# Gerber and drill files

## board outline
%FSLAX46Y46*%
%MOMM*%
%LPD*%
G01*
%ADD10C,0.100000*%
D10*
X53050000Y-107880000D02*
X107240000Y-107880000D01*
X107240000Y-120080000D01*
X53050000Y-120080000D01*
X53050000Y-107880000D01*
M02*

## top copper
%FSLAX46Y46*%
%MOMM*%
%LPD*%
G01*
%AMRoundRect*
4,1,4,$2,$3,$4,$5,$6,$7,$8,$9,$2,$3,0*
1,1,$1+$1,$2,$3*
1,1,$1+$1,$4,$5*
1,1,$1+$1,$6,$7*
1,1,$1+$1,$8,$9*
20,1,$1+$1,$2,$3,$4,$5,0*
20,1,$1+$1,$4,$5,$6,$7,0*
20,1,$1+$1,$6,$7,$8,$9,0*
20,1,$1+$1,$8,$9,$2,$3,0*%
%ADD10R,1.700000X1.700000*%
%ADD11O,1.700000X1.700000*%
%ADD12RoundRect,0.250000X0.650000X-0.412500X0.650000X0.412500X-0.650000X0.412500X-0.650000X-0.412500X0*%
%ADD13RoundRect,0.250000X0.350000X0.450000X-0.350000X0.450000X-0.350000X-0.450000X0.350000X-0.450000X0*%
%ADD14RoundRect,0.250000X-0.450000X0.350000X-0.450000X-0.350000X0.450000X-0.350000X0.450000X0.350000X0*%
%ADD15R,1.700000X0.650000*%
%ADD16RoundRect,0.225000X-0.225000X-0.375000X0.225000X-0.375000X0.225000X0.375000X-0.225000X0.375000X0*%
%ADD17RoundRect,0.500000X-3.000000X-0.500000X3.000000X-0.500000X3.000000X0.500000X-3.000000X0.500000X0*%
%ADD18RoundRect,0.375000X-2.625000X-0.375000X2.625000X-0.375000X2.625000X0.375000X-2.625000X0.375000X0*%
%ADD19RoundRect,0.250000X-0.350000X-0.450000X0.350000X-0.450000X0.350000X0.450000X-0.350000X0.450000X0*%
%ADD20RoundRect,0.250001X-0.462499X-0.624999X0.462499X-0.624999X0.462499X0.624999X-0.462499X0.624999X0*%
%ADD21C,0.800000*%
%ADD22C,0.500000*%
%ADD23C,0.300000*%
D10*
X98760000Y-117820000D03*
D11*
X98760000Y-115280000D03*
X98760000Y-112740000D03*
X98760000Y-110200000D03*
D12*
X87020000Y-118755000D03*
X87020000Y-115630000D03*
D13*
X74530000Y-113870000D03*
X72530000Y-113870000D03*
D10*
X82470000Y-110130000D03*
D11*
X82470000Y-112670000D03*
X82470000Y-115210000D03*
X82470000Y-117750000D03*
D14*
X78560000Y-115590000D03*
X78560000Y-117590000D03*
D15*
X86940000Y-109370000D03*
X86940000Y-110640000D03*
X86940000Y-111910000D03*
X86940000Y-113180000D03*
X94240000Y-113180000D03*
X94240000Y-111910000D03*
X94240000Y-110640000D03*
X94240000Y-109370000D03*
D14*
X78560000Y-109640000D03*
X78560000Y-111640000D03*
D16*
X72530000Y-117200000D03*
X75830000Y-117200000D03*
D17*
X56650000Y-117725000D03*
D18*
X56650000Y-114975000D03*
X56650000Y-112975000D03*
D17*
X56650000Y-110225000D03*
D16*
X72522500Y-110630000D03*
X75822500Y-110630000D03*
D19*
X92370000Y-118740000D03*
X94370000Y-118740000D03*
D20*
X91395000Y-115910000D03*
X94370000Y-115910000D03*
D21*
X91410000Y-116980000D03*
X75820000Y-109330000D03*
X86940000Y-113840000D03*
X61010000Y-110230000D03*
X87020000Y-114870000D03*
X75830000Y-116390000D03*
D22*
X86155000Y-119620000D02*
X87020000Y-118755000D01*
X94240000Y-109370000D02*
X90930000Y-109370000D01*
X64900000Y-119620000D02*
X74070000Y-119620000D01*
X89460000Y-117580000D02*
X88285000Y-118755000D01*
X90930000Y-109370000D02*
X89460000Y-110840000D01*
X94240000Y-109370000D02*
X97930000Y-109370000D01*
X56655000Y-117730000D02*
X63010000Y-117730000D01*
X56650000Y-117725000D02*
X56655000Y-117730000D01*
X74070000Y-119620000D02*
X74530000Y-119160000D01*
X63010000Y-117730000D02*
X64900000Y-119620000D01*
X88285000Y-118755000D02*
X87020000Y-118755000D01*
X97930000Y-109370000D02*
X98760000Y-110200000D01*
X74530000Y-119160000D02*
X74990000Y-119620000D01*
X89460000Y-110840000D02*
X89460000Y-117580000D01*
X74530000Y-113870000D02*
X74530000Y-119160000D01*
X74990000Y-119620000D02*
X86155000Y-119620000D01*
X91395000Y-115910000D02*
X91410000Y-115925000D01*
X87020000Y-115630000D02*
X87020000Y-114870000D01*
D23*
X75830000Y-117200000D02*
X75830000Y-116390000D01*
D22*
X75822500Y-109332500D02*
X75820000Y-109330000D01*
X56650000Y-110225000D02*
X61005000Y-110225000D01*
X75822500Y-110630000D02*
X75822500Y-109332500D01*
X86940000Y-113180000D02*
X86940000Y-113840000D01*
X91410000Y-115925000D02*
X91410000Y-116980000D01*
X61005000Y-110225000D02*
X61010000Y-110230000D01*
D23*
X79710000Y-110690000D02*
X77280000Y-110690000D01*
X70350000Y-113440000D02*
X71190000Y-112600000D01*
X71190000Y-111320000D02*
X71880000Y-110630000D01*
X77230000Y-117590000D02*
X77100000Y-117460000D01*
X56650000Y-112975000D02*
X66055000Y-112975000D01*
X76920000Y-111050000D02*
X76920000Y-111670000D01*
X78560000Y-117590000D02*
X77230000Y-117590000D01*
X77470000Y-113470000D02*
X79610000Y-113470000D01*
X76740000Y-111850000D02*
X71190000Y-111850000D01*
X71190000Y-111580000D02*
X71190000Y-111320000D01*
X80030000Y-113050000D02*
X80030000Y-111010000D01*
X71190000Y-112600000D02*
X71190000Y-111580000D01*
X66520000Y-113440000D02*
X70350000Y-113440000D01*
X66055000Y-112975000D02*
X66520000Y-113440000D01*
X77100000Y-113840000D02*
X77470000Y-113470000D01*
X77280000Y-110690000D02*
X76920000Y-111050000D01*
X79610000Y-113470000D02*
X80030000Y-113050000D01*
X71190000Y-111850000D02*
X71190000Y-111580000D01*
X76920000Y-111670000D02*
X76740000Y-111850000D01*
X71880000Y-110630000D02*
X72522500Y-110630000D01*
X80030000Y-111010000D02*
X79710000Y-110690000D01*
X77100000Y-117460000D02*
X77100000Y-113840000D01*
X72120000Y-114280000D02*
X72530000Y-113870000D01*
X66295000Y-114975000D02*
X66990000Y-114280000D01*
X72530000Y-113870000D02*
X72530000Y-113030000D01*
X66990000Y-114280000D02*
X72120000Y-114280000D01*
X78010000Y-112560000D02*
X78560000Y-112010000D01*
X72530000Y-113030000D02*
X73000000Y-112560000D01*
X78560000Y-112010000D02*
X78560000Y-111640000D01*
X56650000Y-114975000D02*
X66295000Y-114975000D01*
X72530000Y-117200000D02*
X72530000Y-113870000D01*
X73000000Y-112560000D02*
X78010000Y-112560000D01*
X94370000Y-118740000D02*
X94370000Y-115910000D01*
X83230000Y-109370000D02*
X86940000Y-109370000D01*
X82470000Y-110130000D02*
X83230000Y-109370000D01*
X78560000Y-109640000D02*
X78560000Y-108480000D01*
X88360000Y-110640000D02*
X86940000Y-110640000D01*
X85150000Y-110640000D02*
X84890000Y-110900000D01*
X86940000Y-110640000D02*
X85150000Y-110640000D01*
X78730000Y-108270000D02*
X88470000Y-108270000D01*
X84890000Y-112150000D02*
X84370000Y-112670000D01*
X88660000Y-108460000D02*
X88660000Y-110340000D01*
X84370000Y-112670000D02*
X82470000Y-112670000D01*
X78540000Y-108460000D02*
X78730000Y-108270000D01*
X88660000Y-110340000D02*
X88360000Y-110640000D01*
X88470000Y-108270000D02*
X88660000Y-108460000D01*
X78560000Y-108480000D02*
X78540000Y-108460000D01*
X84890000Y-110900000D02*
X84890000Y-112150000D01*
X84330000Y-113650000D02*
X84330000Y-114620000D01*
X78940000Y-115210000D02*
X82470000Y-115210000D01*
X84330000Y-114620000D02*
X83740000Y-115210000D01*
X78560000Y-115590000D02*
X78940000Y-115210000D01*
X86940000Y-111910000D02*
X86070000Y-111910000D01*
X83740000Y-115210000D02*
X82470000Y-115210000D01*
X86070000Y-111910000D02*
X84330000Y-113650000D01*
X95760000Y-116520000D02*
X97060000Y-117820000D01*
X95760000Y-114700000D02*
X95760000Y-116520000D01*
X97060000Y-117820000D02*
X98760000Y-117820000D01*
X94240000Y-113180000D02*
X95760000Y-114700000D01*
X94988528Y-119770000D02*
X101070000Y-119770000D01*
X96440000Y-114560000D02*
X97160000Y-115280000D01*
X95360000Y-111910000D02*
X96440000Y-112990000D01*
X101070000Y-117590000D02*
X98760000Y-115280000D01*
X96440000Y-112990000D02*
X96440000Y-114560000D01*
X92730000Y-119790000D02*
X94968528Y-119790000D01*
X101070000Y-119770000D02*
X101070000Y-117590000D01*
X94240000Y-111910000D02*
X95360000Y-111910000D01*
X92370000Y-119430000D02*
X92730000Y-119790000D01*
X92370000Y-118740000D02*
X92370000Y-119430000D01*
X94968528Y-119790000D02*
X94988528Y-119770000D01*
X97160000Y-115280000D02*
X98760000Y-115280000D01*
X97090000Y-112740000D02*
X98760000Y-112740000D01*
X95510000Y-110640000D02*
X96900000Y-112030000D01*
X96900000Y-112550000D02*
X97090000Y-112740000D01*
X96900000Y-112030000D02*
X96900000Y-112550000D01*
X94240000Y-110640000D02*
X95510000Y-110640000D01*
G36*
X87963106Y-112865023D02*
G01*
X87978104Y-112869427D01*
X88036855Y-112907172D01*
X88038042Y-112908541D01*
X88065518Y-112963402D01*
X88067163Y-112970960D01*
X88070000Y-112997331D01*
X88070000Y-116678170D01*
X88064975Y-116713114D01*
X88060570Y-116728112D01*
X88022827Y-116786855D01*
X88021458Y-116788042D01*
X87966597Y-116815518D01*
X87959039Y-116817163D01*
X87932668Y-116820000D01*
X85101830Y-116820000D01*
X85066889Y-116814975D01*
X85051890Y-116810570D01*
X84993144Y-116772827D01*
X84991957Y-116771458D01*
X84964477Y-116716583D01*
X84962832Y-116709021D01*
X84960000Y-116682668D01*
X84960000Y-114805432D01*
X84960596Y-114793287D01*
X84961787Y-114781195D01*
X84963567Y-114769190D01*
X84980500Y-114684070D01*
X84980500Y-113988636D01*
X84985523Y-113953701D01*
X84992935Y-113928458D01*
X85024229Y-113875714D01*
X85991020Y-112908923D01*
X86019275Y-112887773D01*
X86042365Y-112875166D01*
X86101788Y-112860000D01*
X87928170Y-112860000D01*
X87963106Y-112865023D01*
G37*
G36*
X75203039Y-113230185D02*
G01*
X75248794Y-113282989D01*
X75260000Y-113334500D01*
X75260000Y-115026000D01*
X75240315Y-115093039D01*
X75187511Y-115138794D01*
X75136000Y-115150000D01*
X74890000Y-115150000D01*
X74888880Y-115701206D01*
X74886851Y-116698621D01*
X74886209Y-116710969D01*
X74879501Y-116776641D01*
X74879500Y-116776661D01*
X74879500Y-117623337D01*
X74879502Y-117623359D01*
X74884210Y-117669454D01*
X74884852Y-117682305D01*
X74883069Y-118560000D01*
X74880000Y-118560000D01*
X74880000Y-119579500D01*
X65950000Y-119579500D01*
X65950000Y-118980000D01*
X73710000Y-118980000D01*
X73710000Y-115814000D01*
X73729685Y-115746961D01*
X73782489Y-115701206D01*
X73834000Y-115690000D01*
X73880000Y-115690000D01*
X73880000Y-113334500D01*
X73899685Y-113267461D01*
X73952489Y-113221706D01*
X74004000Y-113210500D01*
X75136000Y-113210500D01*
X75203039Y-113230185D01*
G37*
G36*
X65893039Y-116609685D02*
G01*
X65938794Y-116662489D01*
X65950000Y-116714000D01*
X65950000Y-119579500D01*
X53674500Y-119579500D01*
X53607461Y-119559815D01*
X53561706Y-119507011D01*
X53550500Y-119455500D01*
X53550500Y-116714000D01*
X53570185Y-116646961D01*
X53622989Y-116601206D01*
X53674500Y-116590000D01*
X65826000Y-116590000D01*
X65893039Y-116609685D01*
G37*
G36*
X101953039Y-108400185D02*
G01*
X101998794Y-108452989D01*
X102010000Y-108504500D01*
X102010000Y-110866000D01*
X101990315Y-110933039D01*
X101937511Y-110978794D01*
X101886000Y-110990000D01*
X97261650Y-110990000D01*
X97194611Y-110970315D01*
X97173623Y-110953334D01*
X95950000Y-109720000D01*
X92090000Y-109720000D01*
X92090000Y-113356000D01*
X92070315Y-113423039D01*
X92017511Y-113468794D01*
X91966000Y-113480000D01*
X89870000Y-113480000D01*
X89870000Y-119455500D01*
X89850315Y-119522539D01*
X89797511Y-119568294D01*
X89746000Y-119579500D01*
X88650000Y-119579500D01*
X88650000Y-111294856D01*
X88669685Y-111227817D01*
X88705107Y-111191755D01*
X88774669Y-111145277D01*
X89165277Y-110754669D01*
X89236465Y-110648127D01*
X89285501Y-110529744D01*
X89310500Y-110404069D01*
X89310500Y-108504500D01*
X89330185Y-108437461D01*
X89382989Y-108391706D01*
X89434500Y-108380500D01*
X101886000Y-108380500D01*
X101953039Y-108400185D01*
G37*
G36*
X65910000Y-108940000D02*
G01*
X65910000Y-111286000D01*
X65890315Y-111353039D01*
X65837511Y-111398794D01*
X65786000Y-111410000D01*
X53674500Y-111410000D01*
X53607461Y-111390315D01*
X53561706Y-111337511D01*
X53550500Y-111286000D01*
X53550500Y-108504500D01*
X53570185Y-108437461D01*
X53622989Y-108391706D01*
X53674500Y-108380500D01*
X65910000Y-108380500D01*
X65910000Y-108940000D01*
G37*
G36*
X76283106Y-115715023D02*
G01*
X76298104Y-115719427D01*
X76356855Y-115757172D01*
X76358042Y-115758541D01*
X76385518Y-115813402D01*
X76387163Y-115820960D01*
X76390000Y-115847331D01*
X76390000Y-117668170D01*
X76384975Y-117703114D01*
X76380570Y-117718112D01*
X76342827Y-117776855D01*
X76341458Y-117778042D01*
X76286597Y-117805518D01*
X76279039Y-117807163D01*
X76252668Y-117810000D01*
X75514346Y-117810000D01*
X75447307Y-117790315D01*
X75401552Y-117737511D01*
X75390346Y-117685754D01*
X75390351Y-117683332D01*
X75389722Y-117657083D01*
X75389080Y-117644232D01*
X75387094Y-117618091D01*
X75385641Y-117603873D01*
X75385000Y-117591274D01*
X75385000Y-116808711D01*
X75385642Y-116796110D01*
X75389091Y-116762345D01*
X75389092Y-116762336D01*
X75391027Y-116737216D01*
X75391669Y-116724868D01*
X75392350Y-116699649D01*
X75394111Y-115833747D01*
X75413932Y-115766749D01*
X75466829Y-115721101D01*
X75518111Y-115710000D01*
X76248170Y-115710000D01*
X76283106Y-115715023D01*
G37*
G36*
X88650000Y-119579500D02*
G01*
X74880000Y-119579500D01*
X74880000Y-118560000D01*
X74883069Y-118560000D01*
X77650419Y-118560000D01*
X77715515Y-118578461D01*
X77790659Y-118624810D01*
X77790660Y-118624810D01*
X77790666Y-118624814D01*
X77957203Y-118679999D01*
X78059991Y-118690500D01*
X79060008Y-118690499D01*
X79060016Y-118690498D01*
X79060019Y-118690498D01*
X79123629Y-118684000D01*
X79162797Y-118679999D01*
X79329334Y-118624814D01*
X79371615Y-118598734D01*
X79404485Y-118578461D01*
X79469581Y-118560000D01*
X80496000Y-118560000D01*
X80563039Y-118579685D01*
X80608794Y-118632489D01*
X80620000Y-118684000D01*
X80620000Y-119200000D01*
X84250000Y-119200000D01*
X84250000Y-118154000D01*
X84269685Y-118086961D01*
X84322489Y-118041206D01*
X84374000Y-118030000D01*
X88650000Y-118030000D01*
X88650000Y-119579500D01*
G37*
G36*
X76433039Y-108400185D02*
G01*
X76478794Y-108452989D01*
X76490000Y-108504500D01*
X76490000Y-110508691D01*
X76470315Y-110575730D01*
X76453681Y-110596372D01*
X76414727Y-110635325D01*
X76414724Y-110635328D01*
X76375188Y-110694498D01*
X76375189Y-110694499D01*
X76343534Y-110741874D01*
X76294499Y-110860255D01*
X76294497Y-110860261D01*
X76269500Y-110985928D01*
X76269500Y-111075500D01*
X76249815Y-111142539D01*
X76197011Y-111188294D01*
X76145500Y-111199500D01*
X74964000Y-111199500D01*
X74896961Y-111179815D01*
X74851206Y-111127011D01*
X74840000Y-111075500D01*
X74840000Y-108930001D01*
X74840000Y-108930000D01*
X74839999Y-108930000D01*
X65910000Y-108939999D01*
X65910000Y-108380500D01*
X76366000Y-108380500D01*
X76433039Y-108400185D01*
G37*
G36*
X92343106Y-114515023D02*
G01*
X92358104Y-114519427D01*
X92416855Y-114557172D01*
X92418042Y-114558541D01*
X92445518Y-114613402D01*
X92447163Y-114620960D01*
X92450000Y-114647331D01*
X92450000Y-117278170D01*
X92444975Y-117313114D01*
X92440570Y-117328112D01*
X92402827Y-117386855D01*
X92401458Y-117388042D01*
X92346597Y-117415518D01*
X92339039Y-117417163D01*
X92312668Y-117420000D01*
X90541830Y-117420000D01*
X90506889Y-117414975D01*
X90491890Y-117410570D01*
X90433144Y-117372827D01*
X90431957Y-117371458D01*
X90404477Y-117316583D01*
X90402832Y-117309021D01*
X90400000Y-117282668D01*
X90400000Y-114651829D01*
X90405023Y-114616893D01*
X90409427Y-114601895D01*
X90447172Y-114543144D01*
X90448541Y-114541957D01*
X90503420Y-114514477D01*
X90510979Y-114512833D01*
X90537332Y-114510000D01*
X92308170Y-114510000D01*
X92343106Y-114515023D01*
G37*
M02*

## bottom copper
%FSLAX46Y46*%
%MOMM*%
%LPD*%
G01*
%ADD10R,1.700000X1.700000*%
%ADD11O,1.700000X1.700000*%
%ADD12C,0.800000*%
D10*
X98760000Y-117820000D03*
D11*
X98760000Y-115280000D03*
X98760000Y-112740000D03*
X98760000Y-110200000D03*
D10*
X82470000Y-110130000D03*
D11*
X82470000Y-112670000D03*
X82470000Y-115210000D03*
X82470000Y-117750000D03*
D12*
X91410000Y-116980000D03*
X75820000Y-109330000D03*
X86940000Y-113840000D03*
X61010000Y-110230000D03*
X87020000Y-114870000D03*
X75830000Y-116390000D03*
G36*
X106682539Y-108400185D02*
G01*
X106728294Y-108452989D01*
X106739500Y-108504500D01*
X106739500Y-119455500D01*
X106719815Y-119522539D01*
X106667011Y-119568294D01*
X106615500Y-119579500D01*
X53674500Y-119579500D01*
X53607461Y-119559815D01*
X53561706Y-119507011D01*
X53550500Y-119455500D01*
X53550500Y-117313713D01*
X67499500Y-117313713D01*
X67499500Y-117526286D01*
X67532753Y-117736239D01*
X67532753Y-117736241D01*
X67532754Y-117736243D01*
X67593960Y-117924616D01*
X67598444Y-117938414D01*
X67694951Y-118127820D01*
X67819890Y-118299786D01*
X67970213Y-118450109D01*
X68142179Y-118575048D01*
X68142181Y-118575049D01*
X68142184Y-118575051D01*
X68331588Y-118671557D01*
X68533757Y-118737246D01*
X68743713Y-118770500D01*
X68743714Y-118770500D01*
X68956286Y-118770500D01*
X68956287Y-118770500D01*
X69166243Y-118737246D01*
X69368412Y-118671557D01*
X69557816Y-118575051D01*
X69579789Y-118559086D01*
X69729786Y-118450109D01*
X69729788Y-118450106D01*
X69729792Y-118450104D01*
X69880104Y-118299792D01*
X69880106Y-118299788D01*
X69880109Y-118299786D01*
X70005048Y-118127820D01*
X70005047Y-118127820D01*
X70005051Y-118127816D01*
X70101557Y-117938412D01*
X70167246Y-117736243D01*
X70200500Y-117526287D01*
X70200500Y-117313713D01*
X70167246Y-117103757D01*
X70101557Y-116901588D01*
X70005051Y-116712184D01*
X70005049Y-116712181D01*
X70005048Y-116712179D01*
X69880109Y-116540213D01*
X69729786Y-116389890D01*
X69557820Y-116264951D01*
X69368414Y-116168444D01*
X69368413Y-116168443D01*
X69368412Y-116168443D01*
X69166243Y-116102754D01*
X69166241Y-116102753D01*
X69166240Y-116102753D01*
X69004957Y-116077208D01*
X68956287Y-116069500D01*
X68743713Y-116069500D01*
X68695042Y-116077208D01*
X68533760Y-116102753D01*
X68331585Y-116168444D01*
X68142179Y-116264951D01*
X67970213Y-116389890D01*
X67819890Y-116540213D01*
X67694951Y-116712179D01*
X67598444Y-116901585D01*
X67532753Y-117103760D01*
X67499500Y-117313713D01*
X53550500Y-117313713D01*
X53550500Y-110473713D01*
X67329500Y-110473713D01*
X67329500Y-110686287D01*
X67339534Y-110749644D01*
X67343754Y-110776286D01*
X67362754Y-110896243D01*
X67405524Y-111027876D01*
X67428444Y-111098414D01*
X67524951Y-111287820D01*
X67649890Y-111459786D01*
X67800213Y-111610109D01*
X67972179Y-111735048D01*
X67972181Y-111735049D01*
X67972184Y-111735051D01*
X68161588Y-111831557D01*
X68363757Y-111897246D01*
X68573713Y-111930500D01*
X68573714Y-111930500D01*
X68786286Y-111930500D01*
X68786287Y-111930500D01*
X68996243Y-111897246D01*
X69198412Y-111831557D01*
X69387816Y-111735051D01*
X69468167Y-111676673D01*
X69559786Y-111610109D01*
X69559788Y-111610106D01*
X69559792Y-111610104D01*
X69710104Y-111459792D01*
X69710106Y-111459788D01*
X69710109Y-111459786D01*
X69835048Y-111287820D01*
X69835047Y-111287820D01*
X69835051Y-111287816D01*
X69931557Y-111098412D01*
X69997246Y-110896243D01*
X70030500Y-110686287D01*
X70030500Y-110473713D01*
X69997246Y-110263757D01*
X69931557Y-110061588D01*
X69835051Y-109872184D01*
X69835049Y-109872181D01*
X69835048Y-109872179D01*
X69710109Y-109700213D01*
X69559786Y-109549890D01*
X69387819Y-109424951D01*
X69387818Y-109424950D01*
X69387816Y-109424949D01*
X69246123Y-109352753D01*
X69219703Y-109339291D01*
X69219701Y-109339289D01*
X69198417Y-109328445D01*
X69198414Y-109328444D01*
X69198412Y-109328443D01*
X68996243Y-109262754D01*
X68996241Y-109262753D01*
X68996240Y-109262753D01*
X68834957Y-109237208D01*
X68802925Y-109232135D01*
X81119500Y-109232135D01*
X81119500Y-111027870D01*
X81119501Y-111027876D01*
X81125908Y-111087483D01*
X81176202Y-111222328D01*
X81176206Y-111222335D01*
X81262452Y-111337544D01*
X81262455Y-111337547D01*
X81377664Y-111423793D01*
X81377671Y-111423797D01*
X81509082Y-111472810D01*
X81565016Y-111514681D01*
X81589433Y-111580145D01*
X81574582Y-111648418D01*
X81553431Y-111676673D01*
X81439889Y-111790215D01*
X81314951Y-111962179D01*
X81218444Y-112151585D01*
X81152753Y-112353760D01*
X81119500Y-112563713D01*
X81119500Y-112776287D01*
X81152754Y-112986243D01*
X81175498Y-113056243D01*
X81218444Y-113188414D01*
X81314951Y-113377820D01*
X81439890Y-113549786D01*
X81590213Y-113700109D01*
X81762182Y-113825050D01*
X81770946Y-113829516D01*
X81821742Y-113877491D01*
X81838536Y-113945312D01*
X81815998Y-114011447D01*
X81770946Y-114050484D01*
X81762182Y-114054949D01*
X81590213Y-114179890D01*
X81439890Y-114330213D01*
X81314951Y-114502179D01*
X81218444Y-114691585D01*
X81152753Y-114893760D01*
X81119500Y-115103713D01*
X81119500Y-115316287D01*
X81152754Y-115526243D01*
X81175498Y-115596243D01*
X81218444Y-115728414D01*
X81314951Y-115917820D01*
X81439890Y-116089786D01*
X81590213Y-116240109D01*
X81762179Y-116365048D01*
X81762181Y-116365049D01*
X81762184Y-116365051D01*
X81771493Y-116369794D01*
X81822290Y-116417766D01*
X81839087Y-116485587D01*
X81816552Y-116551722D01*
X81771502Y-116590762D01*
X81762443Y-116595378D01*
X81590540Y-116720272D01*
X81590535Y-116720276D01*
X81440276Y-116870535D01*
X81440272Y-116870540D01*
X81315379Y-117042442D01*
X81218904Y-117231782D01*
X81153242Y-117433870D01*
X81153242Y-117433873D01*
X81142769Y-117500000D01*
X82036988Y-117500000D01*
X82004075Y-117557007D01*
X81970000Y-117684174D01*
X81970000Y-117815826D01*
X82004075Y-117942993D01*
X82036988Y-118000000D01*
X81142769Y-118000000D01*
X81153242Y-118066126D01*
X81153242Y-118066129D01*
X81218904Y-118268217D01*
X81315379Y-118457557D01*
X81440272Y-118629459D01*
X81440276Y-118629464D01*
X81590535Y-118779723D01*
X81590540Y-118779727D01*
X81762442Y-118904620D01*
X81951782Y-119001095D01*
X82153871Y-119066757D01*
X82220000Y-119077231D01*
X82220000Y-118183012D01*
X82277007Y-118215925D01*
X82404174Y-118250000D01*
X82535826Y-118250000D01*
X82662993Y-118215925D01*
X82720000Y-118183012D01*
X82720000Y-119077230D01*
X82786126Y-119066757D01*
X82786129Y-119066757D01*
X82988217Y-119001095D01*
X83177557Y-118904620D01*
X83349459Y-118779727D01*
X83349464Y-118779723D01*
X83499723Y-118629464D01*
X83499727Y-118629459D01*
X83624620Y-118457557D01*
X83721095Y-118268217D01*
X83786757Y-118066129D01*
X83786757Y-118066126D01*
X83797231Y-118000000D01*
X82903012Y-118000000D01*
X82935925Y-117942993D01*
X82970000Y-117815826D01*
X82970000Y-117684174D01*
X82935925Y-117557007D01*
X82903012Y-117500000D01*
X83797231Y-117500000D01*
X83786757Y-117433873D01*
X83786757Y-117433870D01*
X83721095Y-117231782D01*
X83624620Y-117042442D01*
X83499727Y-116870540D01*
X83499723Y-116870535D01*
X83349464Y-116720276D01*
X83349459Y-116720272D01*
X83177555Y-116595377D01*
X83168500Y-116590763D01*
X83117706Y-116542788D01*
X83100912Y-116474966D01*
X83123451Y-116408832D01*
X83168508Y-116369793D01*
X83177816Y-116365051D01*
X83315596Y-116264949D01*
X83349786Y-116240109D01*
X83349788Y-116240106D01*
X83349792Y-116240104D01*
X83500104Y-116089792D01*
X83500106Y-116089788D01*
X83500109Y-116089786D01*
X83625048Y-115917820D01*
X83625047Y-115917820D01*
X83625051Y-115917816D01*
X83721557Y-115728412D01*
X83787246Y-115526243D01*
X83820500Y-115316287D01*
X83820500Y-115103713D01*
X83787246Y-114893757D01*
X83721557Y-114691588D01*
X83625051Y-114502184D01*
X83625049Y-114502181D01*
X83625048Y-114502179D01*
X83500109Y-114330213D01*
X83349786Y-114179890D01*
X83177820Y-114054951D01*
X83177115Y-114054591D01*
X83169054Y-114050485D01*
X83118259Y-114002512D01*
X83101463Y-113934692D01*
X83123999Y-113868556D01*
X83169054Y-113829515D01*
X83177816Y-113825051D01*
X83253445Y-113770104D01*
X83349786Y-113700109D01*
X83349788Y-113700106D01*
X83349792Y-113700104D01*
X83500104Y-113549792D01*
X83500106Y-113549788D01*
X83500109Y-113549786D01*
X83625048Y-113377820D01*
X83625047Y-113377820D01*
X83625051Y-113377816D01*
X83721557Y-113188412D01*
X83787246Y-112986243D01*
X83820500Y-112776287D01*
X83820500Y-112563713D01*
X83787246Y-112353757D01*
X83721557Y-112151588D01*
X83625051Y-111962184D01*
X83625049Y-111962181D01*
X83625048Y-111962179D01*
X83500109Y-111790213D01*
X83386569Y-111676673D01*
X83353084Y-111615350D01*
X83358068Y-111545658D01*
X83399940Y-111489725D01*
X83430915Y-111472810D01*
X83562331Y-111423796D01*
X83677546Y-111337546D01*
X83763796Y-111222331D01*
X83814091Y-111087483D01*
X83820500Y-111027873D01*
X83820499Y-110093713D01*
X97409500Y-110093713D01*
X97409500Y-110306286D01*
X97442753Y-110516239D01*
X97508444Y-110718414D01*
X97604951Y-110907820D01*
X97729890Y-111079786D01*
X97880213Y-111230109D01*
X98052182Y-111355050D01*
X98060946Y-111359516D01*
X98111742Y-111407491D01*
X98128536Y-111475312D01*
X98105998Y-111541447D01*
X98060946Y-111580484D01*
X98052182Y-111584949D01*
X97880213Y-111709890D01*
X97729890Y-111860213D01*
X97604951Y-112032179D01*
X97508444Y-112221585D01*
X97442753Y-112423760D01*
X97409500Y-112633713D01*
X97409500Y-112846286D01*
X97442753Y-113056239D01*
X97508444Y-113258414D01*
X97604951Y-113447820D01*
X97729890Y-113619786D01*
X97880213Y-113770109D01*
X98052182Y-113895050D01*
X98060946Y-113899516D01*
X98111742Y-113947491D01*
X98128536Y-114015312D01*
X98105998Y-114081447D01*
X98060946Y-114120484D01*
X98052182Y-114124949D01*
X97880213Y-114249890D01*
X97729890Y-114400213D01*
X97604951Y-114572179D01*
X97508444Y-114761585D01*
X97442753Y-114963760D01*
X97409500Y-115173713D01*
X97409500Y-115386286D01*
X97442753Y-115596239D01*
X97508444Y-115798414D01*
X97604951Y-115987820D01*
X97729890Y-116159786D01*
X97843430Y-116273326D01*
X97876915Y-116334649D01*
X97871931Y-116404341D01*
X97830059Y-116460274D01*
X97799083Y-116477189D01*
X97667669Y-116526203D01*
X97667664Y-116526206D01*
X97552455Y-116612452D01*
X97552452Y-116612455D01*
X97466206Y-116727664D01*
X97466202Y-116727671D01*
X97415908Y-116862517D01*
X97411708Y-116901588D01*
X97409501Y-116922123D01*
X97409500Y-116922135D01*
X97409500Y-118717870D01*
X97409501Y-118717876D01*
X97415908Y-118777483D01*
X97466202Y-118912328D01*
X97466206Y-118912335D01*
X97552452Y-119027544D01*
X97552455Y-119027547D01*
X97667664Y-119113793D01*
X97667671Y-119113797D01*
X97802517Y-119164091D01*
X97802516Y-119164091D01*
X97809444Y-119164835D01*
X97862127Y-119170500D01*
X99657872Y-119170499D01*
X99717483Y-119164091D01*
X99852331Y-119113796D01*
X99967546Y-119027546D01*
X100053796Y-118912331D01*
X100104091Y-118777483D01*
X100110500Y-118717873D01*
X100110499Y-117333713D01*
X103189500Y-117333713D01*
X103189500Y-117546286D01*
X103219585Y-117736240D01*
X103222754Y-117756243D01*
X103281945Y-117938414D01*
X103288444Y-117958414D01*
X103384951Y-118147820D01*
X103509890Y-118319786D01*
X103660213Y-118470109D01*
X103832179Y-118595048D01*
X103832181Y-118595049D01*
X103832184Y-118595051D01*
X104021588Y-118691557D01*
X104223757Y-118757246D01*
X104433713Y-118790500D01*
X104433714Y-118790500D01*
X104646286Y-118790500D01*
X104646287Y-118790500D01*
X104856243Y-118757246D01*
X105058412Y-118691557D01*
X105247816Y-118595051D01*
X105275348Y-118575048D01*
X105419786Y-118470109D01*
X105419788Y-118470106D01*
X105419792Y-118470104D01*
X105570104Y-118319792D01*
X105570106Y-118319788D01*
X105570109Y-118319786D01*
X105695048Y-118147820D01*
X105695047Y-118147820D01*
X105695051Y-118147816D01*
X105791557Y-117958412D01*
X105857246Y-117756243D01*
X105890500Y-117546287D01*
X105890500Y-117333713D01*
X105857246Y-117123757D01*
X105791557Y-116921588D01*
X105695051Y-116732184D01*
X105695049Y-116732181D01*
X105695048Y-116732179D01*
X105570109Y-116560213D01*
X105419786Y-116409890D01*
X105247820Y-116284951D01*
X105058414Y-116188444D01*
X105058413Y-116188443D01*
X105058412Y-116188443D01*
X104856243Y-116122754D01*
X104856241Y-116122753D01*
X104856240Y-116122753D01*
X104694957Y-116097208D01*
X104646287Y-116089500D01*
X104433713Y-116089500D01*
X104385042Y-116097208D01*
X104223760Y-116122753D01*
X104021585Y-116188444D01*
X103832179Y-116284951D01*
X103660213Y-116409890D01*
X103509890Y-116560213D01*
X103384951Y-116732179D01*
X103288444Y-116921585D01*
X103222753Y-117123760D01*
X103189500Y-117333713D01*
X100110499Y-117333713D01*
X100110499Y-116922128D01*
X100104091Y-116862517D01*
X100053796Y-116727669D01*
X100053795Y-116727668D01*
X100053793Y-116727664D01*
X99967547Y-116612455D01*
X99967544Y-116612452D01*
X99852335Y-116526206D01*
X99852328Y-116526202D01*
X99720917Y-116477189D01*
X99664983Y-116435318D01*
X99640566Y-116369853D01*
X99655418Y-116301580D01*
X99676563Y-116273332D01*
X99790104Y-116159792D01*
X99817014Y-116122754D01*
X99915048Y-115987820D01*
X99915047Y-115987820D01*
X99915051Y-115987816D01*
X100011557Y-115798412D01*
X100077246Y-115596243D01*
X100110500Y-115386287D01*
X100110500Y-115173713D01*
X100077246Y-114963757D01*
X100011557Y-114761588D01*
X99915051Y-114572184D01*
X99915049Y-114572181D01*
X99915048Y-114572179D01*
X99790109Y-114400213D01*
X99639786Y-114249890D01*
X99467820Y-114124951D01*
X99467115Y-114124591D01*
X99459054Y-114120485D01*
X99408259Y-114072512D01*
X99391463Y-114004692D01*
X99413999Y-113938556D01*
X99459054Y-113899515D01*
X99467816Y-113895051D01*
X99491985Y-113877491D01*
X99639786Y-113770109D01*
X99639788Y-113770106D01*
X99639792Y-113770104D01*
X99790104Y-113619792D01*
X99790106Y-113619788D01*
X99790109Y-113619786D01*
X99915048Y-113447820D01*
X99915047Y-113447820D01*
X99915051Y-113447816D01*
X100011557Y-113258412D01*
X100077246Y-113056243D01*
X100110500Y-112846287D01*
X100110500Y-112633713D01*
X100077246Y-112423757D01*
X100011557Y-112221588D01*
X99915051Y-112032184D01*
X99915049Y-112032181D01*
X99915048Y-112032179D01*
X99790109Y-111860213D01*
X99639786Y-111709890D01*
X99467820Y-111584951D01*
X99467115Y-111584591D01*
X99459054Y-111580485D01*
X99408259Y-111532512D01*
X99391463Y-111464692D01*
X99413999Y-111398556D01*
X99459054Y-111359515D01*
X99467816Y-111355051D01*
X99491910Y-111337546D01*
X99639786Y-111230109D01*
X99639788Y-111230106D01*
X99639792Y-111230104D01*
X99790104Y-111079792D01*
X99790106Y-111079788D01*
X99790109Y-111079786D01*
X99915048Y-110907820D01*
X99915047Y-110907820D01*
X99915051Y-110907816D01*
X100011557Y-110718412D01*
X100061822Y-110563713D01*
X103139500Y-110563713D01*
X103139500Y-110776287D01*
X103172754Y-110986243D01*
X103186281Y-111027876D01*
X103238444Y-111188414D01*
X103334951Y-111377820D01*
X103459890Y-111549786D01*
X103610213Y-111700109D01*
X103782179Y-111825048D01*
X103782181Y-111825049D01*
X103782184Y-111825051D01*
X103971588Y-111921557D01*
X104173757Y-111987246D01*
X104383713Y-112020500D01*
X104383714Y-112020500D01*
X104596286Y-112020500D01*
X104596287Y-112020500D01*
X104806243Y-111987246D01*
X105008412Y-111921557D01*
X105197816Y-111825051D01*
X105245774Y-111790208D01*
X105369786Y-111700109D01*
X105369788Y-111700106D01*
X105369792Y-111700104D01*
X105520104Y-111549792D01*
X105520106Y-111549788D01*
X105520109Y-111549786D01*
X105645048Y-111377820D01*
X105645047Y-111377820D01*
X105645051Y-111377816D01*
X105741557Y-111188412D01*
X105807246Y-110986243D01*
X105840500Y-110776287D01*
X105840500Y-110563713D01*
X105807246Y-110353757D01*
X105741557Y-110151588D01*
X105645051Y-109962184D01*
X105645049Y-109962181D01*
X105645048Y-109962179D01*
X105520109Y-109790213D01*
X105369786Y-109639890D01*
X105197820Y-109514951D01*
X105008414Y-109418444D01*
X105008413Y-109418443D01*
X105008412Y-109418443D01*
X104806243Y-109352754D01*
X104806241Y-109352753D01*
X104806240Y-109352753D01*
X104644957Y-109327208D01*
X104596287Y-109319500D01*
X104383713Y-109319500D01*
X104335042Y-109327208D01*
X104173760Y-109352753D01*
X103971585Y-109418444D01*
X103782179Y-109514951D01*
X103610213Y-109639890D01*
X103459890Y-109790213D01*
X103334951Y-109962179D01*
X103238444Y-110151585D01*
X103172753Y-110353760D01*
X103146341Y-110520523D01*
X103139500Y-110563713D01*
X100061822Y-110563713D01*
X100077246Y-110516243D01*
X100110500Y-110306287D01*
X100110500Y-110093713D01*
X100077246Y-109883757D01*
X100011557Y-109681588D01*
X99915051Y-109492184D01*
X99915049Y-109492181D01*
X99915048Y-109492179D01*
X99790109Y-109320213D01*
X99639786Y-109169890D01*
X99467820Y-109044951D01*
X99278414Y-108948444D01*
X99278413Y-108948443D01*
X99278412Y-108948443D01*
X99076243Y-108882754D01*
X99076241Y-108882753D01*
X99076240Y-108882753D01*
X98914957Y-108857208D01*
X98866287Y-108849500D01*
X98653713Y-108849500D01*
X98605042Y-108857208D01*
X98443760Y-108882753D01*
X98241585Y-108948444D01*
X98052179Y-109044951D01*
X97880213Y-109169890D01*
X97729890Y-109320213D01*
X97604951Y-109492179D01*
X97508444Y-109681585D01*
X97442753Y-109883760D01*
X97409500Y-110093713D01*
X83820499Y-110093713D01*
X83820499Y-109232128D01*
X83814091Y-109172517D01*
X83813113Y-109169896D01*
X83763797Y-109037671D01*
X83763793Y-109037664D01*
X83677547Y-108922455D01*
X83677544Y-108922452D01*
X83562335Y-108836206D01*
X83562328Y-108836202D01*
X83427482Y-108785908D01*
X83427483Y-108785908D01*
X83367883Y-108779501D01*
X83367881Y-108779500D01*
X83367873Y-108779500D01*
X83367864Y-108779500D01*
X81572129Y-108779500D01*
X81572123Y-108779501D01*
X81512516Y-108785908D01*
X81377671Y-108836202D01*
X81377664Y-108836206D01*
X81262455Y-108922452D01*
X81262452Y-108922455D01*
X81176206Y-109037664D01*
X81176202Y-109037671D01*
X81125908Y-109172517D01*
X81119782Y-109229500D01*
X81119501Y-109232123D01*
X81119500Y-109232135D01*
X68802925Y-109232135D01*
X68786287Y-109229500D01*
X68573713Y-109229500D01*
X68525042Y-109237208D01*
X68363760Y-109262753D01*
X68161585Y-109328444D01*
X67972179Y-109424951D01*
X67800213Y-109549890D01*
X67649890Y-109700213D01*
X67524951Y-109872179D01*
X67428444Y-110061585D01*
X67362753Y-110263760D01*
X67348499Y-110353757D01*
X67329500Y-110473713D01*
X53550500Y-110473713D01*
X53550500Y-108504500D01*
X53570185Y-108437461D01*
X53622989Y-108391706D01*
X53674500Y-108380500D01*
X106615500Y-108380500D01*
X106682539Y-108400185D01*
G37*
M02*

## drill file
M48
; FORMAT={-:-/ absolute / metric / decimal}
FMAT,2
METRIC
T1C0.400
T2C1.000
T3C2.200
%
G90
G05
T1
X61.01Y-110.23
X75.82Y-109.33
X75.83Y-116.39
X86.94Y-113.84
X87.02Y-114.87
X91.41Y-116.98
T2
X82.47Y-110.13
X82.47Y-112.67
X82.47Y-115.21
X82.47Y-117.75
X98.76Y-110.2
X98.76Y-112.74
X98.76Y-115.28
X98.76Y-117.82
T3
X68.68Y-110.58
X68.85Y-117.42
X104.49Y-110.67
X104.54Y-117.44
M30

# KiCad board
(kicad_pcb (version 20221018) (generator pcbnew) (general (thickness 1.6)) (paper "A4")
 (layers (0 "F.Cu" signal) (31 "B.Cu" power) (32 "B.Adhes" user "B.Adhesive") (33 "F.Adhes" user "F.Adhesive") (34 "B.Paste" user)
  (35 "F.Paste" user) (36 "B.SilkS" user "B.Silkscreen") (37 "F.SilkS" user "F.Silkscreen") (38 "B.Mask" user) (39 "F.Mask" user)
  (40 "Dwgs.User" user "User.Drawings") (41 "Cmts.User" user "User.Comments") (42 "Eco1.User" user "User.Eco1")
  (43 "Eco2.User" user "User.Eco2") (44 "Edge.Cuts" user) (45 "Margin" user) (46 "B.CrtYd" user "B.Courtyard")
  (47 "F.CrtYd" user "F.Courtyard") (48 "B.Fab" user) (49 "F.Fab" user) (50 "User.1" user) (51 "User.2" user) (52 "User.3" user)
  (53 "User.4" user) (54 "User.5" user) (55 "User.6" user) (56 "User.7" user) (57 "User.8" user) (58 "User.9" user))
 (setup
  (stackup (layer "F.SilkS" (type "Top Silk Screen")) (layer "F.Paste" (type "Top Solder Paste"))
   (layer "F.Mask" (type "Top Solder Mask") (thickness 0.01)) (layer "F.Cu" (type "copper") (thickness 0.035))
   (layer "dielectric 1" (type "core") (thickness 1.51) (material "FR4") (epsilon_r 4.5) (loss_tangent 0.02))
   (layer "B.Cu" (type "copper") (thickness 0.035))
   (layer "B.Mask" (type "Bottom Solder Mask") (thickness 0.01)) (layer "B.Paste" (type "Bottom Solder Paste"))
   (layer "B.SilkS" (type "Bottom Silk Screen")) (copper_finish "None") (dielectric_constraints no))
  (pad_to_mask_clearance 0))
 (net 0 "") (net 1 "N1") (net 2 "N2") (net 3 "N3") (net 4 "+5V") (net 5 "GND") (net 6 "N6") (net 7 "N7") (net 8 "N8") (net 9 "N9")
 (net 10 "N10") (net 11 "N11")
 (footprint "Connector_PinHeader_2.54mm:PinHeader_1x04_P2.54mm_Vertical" (layer "F.Cu") (at 98.76 117.82 180)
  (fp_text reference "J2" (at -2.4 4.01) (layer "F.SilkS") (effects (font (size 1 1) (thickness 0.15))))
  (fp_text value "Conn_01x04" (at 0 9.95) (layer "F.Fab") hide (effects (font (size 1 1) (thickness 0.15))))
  (pad "1" thru_hole rect (at 0 0 180) (size 1.7 1.7) (drill 1) (layers "*.Cu" "*.Mask") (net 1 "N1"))
  (pad "2" thru_hole oval (at 0 2.54 180) (size 1.7 1.7) (drill 1) (layers "*.Cu" "*.Mask") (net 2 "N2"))
  (pad "3" thru_hole oval (at 0 5.08 180) (size 1.7 1.7) (drill 1) (layers "*.Cu" "*.Mask") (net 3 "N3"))
  (pad "4" thru_hole oval (at 0 7.62 180) (size 1.7 1.7) (drill 1) (layers "*.Cu" "*.Mask") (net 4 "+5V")))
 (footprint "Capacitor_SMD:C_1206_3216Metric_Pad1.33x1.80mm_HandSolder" (layer "F.Cu") (at 87.02 117.1925 90)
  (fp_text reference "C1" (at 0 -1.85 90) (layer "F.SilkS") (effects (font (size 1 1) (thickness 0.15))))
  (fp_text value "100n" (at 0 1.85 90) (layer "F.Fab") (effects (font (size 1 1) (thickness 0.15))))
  (pad "1" smd roundrect (at -1.5625 0 90) (size 1.325 1.8) (layers "F.Cu" "F.Paste" "F.Mask") (roundrect_rratio 0.1886792453) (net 4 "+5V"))
  (pad "2" smd roundrect (at 1.5625 0 90) (size 1.325 1.8) (layers "F.Cu" "F.Paste" "F.Mask") (roundrect_rratio 0.1886792453) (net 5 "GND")))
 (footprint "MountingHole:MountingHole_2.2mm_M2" (layer "F.Cu") (at 104.54 117.44)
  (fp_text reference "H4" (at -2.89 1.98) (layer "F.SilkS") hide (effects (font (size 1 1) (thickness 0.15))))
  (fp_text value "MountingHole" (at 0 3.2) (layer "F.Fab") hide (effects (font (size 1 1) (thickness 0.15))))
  (pad "" np_thru_hole circle (at 0 0) (size 2.2 2.2) (drill 2.2) (layers "*.Cu" "*.Mask")))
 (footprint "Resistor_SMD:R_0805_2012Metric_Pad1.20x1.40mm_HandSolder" (layer "F.Cu") (at 73.53 113.87 180)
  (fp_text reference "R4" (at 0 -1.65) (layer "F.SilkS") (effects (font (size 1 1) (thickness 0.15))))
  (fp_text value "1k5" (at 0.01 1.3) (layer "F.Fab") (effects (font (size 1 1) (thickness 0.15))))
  (pad "1" smd roundrect (at -1 0 180) (size 1.2 1.4) (layers "F.Cu" "F.Paste" "F.Mask") (roundrect_rratio 0.2083333333) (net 4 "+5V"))
  (pad "2" smd roundrect (at 1 0 180) (size 1.2 1.4) (layers "F.Cu" "F.Paste" "F.Mask") (roundrect_rratio 0.2083333333) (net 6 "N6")))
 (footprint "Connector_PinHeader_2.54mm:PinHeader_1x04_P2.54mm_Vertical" (layer "F.Cu") (at 82.47 110.13)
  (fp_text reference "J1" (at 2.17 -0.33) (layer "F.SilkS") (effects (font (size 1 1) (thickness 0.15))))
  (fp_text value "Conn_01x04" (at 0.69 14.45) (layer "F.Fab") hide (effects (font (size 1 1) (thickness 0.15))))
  (pad "1" thru_hole rect (at 0 0) (size 1.7 1.7) (drill 1) (layers "*.Cu" "*.Mask") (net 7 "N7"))
  (pad "2" thru_hole oval (at 0 2.54) (size 1.7 1.7) (drill 1) (layers "*.Cu" "*.Mask") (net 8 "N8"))
  (pad "3" thru_hole oval (at 0 5.08) (size 1.7 1.7) (drill 1) (layers "*.Cu" "*.Mask") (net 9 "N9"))
  (pad "4" thru_hole oval (at 0 7.62) (size 1.7 1.7) (drill 1) (layers "*.Cu" "*.Mask") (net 5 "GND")))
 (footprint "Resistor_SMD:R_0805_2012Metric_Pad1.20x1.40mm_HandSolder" (layer "F.Cu") (at 78.56 116.59 -90)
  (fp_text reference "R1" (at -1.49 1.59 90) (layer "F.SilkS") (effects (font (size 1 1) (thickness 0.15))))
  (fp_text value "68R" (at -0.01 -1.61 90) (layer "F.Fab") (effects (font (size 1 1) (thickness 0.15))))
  (pad "1" smd roundrect (at -1 0 270) (size 1.2 1.4) (layers "F.Cu" "F.Paste" "F.Mask") (roundrect_rratio 0.2083333333) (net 9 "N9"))
  (pad "2" smd roundrect (at 1 0 270) (size 1.2 1.4) (layers "F.Cu" "F.Paste" "F.Mask") (roundrect_rratio 0.2083333333) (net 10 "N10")))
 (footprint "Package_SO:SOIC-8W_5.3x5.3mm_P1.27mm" (layer "F.Cu") (at 90.59 111.275)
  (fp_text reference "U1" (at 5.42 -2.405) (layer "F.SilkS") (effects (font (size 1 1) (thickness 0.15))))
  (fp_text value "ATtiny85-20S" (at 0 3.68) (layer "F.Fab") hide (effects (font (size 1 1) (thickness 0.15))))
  (pad "1" smd rect (at -3.65 -1.905) (size 1.7 0.65) (layers "F.Cu" "F.Paste" "F.Mask") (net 7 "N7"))
  (pad "2" smd rect (at -3.65 -0.635) (size 1.7 0.65) (layers "F.Cu" "F.Paste" "F.Mask") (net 8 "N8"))
  (pad "3" smd rect (at -3.65 0.635) (size 1.7 0.65) (layers "F.Cu" "F.Paste" "F.Mask") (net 9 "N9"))
  (pad "4" smd rect (at -3.65 1.905) (size 1.7 0.65) (layers "F.Cu" "F.Paste" "F.Mask") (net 5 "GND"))
  (pad "5" smd rect (at 3.65 1.905) (size 1.7 0.65) (layers "F.Cu" "F.Paste" "F.Mask") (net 1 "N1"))
  (pad "6" smd rect (at 3.65 0.635) (size 1.7 0.65) (layers "F.Cu" "F.Paste" "F.Mask") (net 2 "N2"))
  (pad "7" smd rect (at 3.65 -0.635) (size 1.7 0.65) (layers "F.Cu" "F.Paste" "F.Mask") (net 3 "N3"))
  (pad "8" smd rect (at 3.65 -1.905) (size 1.7 0.65) (layers "F.Cu" "F.Paste" "F.Mask") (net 4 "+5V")))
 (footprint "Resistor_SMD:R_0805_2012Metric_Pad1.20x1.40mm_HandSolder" (layer "F.Cu") (at 78.56 110.64 -90)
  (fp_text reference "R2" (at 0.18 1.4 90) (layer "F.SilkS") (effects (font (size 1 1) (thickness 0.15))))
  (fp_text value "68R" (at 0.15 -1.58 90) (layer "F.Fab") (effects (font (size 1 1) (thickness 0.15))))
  (pad "1" smd roundrect (at -1 0 270) (size 1.2 1.4) (layers "F.Cu" "F.Paste" "F.Mask") (roundrect_rratio 0.2083333333) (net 8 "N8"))
  (pad "2" smd roundrect (at 1 0 270) (size 1.2 1.4) (layers "F.Cu" "F.Paste" "F.Mask") (roundrect_rratio 0.2083333333) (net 6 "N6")))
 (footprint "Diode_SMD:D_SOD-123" (layer "F.Cu") (at 74.18 117.2)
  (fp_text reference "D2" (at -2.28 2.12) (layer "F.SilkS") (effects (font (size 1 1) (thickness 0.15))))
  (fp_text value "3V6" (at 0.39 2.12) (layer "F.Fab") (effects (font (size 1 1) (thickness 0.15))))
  (pad "1" smd roundrect (at -1.65 0) (size 0.9 1.2) (layers "F.Cu" "F.Paste" "F.Mask") (roundrect_rratio 0.25) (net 6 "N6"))
  (pad "2" smd roundrect (at 1.65 0) (size 0.9 1.2) (layers "F.Cu" "F.Paste" "F.Mask") (roundrect_rratio 0.25) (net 5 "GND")))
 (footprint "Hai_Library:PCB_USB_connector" (layer "F.Cu") (at 56.65 113.975)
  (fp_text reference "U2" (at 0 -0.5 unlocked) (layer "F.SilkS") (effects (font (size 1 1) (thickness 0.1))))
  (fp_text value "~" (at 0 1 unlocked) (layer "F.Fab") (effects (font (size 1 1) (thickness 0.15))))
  (pad "1" smd roundrect (at 0 3.75) (size 7 2) (layers "F.Cu" "F.Paste" "F.Mask") (roundrect_rratio 0.25) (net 4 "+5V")
   (thermal_bridge_angle 45))
  (pad "2" smd roundrect (at 0 1) (size 6 1.5) (layers "F.Cu" "F.Paste" "F.Mask") (roundrect_rratio 0.25) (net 6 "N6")
   (thermal_bridge_angle 45))
  (pad "3" smd roundrect (at 0 -1) (size 6 1.5) (layers "F.Cu" "F.Paste" "F.Mask") (roundrect_rratio 0.25) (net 10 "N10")
   (thermal_bridge_angle 45))
  (pad "4" smd roundrect (at 0 -3.75) (size 7 2) (layers "F.Cu" "F.Paste" "F.Mask") (roundrect_rratio 0.25) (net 5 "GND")
   (thermal_bridge_angle 45)))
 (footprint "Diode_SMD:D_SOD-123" (layer "F.Cu") (at 74.1725 110.63)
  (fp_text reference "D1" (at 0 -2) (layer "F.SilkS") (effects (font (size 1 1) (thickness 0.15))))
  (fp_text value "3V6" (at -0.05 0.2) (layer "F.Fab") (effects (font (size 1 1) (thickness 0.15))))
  (pad "1" smd roundrect (at -1.65 0) (size 0.9 1.2) (layers "F.Cu" "F.Paste" "F.Mask") (roundrect_rratio 0.25) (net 10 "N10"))
  (pad "2" smd roundrect (at 1.65 0) (size 0.9 1.2) (layers "F.Cu" "F.Paste" "F.Mask") (roundrect_rratio 0.25) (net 5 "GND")))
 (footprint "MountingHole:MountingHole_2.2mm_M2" (layer "F.Cu") (at 68.68 110.58)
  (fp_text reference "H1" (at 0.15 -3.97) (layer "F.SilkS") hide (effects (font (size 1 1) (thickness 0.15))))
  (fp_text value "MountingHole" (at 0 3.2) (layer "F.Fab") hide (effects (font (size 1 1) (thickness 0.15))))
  (pad "" np_thru_hole circle (at 0 0) (size 2.2 2.2) (drill 2.2) (layers "*.Cu" "*.Mask")))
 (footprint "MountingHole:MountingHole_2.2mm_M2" (layer "F.Cu") (at 68.85 117.42)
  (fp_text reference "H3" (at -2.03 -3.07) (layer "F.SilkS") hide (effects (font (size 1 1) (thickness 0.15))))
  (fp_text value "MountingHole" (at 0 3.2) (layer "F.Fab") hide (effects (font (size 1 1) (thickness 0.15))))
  (pad "" np_thru_hole circle (at 0 0) (size 2.2 2.2) (drill 2.2) (layers "*.Cu" "*.Mask")))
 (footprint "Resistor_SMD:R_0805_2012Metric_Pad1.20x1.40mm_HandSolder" (layer "F.Cu") (at 93.37 118.74)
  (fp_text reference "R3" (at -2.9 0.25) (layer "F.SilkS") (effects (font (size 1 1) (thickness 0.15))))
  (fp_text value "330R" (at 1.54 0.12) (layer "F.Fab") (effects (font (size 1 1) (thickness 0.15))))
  (pad "1" smd roundrect (at -1 0) (size 1.2 1.4) (layers "F.Cu" "F.Paste" "F.Mask") (roundrect_rratio 0.2083333333) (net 2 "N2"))
  (pad "2" smd roundrect (at 1 0) (size 1.2 1.4) (layers "F.Cu" "F.Paste" "F.Mask") (roundrect_rratio 0.2083333333) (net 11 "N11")))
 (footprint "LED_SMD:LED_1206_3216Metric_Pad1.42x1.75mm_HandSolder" (layer "F.Cu") (at 92.8825 115.91)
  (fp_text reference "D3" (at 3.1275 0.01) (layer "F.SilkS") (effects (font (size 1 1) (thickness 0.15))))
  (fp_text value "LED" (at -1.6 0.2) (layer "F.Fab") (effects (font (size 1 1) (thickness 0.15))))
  (pad "1" smd roundrect (at -1.4875 0) (size 1.425 1.75) (layers "F.Cu" "F.Paste" "F.Mask") (roundrect_rratio 0.1754392982) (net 5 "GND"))
  (pad "2" smd roundrect (at 1.4875 0) (size 1.425 1.75) (layers "F.Cu" "F.Paste" "F.Mask") (roundrect_rratio 0.1754392982) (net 11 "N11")))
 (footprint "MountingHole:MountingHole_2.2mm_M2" (layer "F.Cu") (at 104.49 110.67)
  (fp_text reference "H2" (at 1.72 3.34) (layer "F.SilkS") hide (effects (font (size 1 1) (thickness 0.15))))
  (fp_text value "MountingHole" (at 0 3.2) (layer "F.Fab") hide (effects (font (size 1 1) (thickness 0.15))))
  (pad "" np_thru_hole circle (at 0 0) (size 2.2 2.2) (drill 2.2) (layers "*.Cu" "*.Mask")))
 (gr_rect (start 53.05 107.88) (end 107.24 120.08) (stroke (width 0.1) (type default)) (fill none) (layer "Edge.Cuts"))
 (segment (start 86.155 119.62) (end 87.02 118.755) (width 0.5) (layer "F.Cu") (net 4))
 (segment (start 94.24 109.37) (end 90.93 109.37) (width 0.5) (layer "F.Cu") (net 4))
 (segment (start 64.9 119.62) (end 74.07 119.62) (width 0.5) (layer "F.Cu") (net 4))
 (segment (start 89.46 117.58) (end 88.285 118.755) (width 0.5) (layer "F.Cu") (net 4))
 (segment (start 90.93 109.37) (end 89.46 110.84) (width 0.5) (layer "F.Cu") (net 4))
 (segment (start 94.24 109.37) (end 97.93 109.37) (width 0.5) (layer "F.Cu") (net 4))
 (segment (start 56.655 117.73) (end 63.01 117.73) (width 0.5) (layer "F.Cu") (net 4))
 (segment (start 56.65 117.725) (end 56.655 117.73) (width 0.5) (layer "F.Cu") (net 4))
 (segment (start 74.07 119.62) (end 74.53 119.16) (width 0.5) (layer "F.Cu") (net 4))
 (segment (start 63.01 117.73) (end 64.9 119.62) (width 0.5) (layer "F.Cu") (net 4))
 (segment (start 88.285 118.755) (end 87.02 118.755) (width 0.5) (layer "F.Cu") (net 4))
 (segment (start 97.93 109.37) (end 98.76 110.2) (width 0.5) (layer "F.Cu") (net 4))
 (segment (start 74.53 119.16) (end 74.99 119.62) (width 0.5) (layer "F.Cu") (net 4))
 (segment (start 89.46 110.84) (end 89.46 117.58) (width 0.5) (layer "F.Cu") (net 4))
 (segment (start 74.53 113.87) (end 74.53 119.16) (width 0.5) (layer "F.Cu") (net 4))
 (segment (start 74.99 119.62) (end 86.155 119.62) (width 0.5) (layer "F.Cu") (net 4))
 (segment (start 91.395 115.91) (end 91.41 115.925) (width 0.5) (layer "F.Cu") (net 5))
 (segment (start 87.02 115.63) (end 87.02 114.87) (width 0.5) (layer "F.Cu") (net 5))
 (segment (start 75.83 117.2) (end 75.83 116.39) (width 0.3) (layer "F.Cu") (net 5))
 (segment (start 75.8225 109.3325) (end 75.82 109.33) (width 0.5) (layer "F.Cu") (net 5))
 (segment (start 56.65 110.225) (end 61.005 110.225) (width 0.5) (layer "F.Cu") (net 5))
 (segment (start 75.8225 110.63) (end 75.8225 109.3325) (width 0.5) (layer "F.Cu") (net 5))
 (segment (start 86.94 113.18) (end 86.94 113.84) (width 0.5) (layer "F.Cu") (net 5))
 (segment (start 91.41 115.925) (end 91.41 116.98) (width 0.5) (layer "F.Cu") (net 5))
 (segment (start 61.005 110.225) (end 61.01 110.23) (width 0.5) (layer "F.Cu") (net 5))
 (via (at 91.41 116.98) (size 0.8) (drill 0.4) (layers "F.Cu" "B.Cu") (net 5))
 (via (at 75.82 109.33) (size 0.8) (drill 0.4) (layers "F.Cu" "B.Cu") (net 5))
 (via (at 86.94 113.84) (size 0.8) (drill 0.4) (layers "F.Cu" "B.Cu") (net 5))
 (via (at 61.01 110.23) (size 0.8) (drill 0.4) (layers "F.Cu" "B.Cu") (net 5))
 (via (at 87.02 114.87) (size 0.8) (drill 0.4) (layers "F.Cu" "B.Cu") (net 5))
 (via (at 75.83 116.39) (size 0.8) (drill 0.4) (layers "F.Cu" "B.Cu") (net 5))
 (segment (start 79.71 110.69) (end 77.28 110.69) (width 0.3) (layer "F.Cu") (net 10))
 (segment (start 70.35 113.44) (end 71.19 112.6) (width 0.3) (layer "F.Cu") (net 10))
 (segment (start 71.19 111.32) (end 71.88 110.63) (width 0.3) (layer "F.Cu") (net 10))
 (segment (start 77.23 117.59) (end 77.1 117.46) (width 0.3) (layer "F.Cu") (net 10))
 (segment (start 56.65 112.975) (end 66.055 112.975) (width 0.3) (layer "F.Cu") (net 10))
 (segment (start 76.92 111.05) (end 76.92 111.67) (width 0.3) (layer "F.Cu") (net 10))
 (segment (start 78.56 117.59) (end 77.23 117.59) (width 0.3) (layer "F.Cu") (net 10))
 (segment (start 77.47 113.47) (end 79.61 113.47) (width 0.3) (layer "F.Cu") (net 10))
 (segment (start 76.74 111.85) (end 71.19 111.85) (width 0.3) (layer "F.Cu") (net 10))
 (segment (start 71.19 111.58) (end 71.19 111.32) (width 0.3) (layer "F.Cu") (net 10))
 (segment (start 80.03 113.05) (end 80.03 111.01) (width 0.3) (layer "F.Cu") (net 10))
 (segment (start 71.19 112.6) (end 71.19 111.58) (width 0.3) (layer "F.Cu") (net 10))
 (segment (start 66.52 113.44) (end 70.35 113.44) (width 0.3) (layer "F.Cu") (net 10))
 (segment (start 66.055 112.975) (end 66.52 113.44) (width 0.3) (layer "F.Cu") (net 10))
 (segment (start 77.1 113.84) (end 77.47 113.47) (width 0.3) (layer "F.Cu") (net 10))
 (segment (start 77.28 110.69) (end 76.92 111.05) (width 0.3) (layer "F.Cu") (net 10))
 (segment (start 79.61 113.47) (end 80.03 113.05) (width 0.3) (layer "F.Cu") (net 10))
 (segment (start 71.19 111.85) (end 71.19 111.58) (width 0.3) (layer "F.Cu") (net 10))
 (segment (start 76.92 111.67) (end 76.74 111.85) (width 0.3) (layer "F.Cu") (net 10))
 (segment (start 71.88 110.63) (end 72.5225 110.63) (width 0.3) (layer "F.Cu") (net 10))
 (segment (start 80.03 111.01) (end 79.71 110.69) (width 0.3) (layer "F.Cu") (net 10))
 (segment (start 77.1 117.46) (end 77.1 113.84) (width 0.3) (layer "F.Cu") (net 10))
 (segment (start 72.12 114.28) (end 72.53 113.87) (width 0.3) (layer "F.Cu") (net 6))
 (segment (start 66.295 114.975) (end 66.99 114.28) (width 0.3) (layer "F.Cu") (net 6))
 (segment (start 72.53 113.87) (end 72.53 113.03) (width 0.3) (layer "F.Cu") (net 6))
 (segment (start 66.99 114.28) (end 72.12 114.28) (width 0.3) (layer "F.Cu") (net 6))
 (segment (start 78.01 112.56) (end 78.56 112.01) (width 0.3) (layer "F.Cu") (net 6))
 (segment (start 72.53 113.03) (end 73 112.56) (width 0.3) (layer "F.Cu") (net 6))
 (segment (start 78.56 112.01) (end 78.56 111.64) (width 0.3) (layer "F.Cu") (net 6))
 (segment (start 56.65 114.975) (end 66.295 114.975) (width 0.3) (layer "F.Cu") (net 6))
 (segment (start 72.53 117.2) (end 72.53 113.87) (width 0.3) (layer "F.Cu") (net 6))
 (segment (start 73 112.56) (end 78.01 112.56) (width 0.3) (layer "F.Cu") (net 6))
 (segment (start 94.37 118.74) (end 94.37 115.91) (width 0.3) (layer "F.Cu") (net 11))
 (segment (start 83.23 109.37) (end 86.94 109.37) (width 0.3) (layer "F.Cu") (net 7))
 (segment (start 82.47 110.13) (end 83.23 109.37) (width 0.3) (layer "F.Cu") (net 7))
 (segment (start 78.56 109.64) (end 78.56 108.48) (width 0.3) (layer "F.Cu") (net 8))
 (segment (start 88.36 110.64) (end 86.94 110.64) (width 0.3) (layer "F.Cu") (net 8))
 (segment (start 85.15 110.64) (end 84.89 110.9) (width 0.3) (layer "F.Cu") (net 8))
 (segment (start 86.94 110.64) (end 85.15 110.64) (width 0.3) (layer "F.Cu") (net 8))
 (segment (start 78.73 108.27) (end 88.47 108.27) (width 0.3) (layer "F.Cu") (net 8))
 (segment (start 84.89 112.15) (end 84.37 112.67) (width 0.3) (layer "F.Cu") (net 8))
 (segment (start 88.66 108.46) (end 88.66 110.34) (width 0.3) (layer "F.Cu") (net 8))
 (segment (start 84.37 112.67) (end 82.47 112.67) (width 0.3) (layer "F.Cu") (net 8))
 (segment (start 78.54 108.46) (end 78.73 108.27) (width 0.3) (layer "F.Cu") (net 8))
 (segment (start 88.66 110.34) (end 88.36 110.64) (width 0.3) (layer "F.Cu") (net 8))
 (segment (start 88.47 108.27) (end 88.66 108.46) (width 0.3) (layer "F.Cu") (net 8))
 (segment (start 78.56 108.48) (end 78.54 108.46) (width 0.3) (layer "F.Cu") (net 8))
 (segment (start 84.89 110.9) (end 84.89 112.15) (width 0.3) (layer "F.Cu") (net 8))
 (segment (start 84.33 113.65) (end 84.33 114.62) (width 0.3) (layer "F.Cu") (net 9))
 (segment (start 78.94 115.21) (end 82.47 115.21) (width 0.3) (layer "F.Cu") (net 9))
 (segment (start 84.33 114.62) (end 83.74 115.21) (width 0.3) (layer "F.Cu") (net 9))
 (segment (start 78.56 115.59) (end 78.94 115.21) (width 0.3) (layer "F.Cu") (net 9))
 (segment (start 86.94 111.91) (end 86.07 111.91) (width 0.3) (layer "F.Cu") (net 9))
 (segment (start 83.74 115.21) (end 82.47 115.21) (width 0.3) (layer "F.Cu") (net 9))
 (segment (start 86.07 111.91) (end 84.33 113.65) (width 0.3) (layer "F.Cu") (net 9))
 (segment (start 95.76 116.52) (end 97.06 117.82) (width 0.3) (layer "F.Cu") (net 1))
 (segment (start 95.76 114.7) (end 95.76 116.52) (width 0.3) (layer "F.Cu") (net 1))
 (segment (start 97.06 117.82) (end 98.76 117.82) (width 0.3) (layer "F.Cu") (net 1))
 (segment (start 94.24 113.18) (end 95.76 114.7) (width 0.3) (layer "F.Cu") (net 1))
 (segment (start 94.988528 119.77) (end 101.07 119.77) (width 0.3) (layer "F.Cu") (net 2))
 (segment (start 96.44 114.56) (end 97.16 115.28) (width 0.3) (layer "F.Cu") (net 2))
 (segment (start 95.36 111.91) (end 96.44 112.99) (width 0.3) (layer "F.Cu") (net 2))
 (segment (start 101.07 117.59) (end 98.76 115.28) (width 0.3) (layer "F.Cu") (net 2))
 (segment (start 96.44 112.99) (end 96.44 114.56) (width 0.3) (layer "F.Cu") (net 2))
 (segment (start 92.73 119.79) (end 94.968528 119.79) (width 0.3) (layer "F.Cu") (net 2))
 (segment (start 101.07 119.77) (end 101.07 117.59) (width 0.3) (layer "F.Cu") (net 2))
 (segment (start 94.24 111.91) (end 95.36 111.91) (width 0.3) (layer "F.Cu") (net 2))
 (segment (start 92.37 119.43) (end 92.73 119.79) (width 0.3) (layer "F.Cu") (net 2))
 (segment (start 92.37 118.74) (end 92.37 119.43) (width 0.3) (layer "F.Cu") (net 2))
 (segment (start 94.968528 119.79) (end 94.988528 119.77) (width 0.3) (layer "F.Cu") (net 2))
 (segment (start 97.16 115.28) (end 98.76 115.28) (width 0.3) (layer "F.Cu") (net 2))
 (segment (start 97.09 112.74) (end 98.76 112.74) (width 0.3) (layer "F.Cu") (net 3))
 (segment (start 95.51 110.64) (end 96.9 112.03) (width 0.3) (layer "F.Cu") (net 3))
 (segment (start 96.9 112.55) (end 97.09 112.74) (width 0.3) (layer "F.Cu") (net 3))
 (segment (start 96.9 112.03) (end 96.9 112.55) (width 0.3) (layer "F.Cu") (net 3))
 (segment (start 94.24 110.64) (end 95.51 110.64) (width 0.3) (layer "F.Cu") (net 3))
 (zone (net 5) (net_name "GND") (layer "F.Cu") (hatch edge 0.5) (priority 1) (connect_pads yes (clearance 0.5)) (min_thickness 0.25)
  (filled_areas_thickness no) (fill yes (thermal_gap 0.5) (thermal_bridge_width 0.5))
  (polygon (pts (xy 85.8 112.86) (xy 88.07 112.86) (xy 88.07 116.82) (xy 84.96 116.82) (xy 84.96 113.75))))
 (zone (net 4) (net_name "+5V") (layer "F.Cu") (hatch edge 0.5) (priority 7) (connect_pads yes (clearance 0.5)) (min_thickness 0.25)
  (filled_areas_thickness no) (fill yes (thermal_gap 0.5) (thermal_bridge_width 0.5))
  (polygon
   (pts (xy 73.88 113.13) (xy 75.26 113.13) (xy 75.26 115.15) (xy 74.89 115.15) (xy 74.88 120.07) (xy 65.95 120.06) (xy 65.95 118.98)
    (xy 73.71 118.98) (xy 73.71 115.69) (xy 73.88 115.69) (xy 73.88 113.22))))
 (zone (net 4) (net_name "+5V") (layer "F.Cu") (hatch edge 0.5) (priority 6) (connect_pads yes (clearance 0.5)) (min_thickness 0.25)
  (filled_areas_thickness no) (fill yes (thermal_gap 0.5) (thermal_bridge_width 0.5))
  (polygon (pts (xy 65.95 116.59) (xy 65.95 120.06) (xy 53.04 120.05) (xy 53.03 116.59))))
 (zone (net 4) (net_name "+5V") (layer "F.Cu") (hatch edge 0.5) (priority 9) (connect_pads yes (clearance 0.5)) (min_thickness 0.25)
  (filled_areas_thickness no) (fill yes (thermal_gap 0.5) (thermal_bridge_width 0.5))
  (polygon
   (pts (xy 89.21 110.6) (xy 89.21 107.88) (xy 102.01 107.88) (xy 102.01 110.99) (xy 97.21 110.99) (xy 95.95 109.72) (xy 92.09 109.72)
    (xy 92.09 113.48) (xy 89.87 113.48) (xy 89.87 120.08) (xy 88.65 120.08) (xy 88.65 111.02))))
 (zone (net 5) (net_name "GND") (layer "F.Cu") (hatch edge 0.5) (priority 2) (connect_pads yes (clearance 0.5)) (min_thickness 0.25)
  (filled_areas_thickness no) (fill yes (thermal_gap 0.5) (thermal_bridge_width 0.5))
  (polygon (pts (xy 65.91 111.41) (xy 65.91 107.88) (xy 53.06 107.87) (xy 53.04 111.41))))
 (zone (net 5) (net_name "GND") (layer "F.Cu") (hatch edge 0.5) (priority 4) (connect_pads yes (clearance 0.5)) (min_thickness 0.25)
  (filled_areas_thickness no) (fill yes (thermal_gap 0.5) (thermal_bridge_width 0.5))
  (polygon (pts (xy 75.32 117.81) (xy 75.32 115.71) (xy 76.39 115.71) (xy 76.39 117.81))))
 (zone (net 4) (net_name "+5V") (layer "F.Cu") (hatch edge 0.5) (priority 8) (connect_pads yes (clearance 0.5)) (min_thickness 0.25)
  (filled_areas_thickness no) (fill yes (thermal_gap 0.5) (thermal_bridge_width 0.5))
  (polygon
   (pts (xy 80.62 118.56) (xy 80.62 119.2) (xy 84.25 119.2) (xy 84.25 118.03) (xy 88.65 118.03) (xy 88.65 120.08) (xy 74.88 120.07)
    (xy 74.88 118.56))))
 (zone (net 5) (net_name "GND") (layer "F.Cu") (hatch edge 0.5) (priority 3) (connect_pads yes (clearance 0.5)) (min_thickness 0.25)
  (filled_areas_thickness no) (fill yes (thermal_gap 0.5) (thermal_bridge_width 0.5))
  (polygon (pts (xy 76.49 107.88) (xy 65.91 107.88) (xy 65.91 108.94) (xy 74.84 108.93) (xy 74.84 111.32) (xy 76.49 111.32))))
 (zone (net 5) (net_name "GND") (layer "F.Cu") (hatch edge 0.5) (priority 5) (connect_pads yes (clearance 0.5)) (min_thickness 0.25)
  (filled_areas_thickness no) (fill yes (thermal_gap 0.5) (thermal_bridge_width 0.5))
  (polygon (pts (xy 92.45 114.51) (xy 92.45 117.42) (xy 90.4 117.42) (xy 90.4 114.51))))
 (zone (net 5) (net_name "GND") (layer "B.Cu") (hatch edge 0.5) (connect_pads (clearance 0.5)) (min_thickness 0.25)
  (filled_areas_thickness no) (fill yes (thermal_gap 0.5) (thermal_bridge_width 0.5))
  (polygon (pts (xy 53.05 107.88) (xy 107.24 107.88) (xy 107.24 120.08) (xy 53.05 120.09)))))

